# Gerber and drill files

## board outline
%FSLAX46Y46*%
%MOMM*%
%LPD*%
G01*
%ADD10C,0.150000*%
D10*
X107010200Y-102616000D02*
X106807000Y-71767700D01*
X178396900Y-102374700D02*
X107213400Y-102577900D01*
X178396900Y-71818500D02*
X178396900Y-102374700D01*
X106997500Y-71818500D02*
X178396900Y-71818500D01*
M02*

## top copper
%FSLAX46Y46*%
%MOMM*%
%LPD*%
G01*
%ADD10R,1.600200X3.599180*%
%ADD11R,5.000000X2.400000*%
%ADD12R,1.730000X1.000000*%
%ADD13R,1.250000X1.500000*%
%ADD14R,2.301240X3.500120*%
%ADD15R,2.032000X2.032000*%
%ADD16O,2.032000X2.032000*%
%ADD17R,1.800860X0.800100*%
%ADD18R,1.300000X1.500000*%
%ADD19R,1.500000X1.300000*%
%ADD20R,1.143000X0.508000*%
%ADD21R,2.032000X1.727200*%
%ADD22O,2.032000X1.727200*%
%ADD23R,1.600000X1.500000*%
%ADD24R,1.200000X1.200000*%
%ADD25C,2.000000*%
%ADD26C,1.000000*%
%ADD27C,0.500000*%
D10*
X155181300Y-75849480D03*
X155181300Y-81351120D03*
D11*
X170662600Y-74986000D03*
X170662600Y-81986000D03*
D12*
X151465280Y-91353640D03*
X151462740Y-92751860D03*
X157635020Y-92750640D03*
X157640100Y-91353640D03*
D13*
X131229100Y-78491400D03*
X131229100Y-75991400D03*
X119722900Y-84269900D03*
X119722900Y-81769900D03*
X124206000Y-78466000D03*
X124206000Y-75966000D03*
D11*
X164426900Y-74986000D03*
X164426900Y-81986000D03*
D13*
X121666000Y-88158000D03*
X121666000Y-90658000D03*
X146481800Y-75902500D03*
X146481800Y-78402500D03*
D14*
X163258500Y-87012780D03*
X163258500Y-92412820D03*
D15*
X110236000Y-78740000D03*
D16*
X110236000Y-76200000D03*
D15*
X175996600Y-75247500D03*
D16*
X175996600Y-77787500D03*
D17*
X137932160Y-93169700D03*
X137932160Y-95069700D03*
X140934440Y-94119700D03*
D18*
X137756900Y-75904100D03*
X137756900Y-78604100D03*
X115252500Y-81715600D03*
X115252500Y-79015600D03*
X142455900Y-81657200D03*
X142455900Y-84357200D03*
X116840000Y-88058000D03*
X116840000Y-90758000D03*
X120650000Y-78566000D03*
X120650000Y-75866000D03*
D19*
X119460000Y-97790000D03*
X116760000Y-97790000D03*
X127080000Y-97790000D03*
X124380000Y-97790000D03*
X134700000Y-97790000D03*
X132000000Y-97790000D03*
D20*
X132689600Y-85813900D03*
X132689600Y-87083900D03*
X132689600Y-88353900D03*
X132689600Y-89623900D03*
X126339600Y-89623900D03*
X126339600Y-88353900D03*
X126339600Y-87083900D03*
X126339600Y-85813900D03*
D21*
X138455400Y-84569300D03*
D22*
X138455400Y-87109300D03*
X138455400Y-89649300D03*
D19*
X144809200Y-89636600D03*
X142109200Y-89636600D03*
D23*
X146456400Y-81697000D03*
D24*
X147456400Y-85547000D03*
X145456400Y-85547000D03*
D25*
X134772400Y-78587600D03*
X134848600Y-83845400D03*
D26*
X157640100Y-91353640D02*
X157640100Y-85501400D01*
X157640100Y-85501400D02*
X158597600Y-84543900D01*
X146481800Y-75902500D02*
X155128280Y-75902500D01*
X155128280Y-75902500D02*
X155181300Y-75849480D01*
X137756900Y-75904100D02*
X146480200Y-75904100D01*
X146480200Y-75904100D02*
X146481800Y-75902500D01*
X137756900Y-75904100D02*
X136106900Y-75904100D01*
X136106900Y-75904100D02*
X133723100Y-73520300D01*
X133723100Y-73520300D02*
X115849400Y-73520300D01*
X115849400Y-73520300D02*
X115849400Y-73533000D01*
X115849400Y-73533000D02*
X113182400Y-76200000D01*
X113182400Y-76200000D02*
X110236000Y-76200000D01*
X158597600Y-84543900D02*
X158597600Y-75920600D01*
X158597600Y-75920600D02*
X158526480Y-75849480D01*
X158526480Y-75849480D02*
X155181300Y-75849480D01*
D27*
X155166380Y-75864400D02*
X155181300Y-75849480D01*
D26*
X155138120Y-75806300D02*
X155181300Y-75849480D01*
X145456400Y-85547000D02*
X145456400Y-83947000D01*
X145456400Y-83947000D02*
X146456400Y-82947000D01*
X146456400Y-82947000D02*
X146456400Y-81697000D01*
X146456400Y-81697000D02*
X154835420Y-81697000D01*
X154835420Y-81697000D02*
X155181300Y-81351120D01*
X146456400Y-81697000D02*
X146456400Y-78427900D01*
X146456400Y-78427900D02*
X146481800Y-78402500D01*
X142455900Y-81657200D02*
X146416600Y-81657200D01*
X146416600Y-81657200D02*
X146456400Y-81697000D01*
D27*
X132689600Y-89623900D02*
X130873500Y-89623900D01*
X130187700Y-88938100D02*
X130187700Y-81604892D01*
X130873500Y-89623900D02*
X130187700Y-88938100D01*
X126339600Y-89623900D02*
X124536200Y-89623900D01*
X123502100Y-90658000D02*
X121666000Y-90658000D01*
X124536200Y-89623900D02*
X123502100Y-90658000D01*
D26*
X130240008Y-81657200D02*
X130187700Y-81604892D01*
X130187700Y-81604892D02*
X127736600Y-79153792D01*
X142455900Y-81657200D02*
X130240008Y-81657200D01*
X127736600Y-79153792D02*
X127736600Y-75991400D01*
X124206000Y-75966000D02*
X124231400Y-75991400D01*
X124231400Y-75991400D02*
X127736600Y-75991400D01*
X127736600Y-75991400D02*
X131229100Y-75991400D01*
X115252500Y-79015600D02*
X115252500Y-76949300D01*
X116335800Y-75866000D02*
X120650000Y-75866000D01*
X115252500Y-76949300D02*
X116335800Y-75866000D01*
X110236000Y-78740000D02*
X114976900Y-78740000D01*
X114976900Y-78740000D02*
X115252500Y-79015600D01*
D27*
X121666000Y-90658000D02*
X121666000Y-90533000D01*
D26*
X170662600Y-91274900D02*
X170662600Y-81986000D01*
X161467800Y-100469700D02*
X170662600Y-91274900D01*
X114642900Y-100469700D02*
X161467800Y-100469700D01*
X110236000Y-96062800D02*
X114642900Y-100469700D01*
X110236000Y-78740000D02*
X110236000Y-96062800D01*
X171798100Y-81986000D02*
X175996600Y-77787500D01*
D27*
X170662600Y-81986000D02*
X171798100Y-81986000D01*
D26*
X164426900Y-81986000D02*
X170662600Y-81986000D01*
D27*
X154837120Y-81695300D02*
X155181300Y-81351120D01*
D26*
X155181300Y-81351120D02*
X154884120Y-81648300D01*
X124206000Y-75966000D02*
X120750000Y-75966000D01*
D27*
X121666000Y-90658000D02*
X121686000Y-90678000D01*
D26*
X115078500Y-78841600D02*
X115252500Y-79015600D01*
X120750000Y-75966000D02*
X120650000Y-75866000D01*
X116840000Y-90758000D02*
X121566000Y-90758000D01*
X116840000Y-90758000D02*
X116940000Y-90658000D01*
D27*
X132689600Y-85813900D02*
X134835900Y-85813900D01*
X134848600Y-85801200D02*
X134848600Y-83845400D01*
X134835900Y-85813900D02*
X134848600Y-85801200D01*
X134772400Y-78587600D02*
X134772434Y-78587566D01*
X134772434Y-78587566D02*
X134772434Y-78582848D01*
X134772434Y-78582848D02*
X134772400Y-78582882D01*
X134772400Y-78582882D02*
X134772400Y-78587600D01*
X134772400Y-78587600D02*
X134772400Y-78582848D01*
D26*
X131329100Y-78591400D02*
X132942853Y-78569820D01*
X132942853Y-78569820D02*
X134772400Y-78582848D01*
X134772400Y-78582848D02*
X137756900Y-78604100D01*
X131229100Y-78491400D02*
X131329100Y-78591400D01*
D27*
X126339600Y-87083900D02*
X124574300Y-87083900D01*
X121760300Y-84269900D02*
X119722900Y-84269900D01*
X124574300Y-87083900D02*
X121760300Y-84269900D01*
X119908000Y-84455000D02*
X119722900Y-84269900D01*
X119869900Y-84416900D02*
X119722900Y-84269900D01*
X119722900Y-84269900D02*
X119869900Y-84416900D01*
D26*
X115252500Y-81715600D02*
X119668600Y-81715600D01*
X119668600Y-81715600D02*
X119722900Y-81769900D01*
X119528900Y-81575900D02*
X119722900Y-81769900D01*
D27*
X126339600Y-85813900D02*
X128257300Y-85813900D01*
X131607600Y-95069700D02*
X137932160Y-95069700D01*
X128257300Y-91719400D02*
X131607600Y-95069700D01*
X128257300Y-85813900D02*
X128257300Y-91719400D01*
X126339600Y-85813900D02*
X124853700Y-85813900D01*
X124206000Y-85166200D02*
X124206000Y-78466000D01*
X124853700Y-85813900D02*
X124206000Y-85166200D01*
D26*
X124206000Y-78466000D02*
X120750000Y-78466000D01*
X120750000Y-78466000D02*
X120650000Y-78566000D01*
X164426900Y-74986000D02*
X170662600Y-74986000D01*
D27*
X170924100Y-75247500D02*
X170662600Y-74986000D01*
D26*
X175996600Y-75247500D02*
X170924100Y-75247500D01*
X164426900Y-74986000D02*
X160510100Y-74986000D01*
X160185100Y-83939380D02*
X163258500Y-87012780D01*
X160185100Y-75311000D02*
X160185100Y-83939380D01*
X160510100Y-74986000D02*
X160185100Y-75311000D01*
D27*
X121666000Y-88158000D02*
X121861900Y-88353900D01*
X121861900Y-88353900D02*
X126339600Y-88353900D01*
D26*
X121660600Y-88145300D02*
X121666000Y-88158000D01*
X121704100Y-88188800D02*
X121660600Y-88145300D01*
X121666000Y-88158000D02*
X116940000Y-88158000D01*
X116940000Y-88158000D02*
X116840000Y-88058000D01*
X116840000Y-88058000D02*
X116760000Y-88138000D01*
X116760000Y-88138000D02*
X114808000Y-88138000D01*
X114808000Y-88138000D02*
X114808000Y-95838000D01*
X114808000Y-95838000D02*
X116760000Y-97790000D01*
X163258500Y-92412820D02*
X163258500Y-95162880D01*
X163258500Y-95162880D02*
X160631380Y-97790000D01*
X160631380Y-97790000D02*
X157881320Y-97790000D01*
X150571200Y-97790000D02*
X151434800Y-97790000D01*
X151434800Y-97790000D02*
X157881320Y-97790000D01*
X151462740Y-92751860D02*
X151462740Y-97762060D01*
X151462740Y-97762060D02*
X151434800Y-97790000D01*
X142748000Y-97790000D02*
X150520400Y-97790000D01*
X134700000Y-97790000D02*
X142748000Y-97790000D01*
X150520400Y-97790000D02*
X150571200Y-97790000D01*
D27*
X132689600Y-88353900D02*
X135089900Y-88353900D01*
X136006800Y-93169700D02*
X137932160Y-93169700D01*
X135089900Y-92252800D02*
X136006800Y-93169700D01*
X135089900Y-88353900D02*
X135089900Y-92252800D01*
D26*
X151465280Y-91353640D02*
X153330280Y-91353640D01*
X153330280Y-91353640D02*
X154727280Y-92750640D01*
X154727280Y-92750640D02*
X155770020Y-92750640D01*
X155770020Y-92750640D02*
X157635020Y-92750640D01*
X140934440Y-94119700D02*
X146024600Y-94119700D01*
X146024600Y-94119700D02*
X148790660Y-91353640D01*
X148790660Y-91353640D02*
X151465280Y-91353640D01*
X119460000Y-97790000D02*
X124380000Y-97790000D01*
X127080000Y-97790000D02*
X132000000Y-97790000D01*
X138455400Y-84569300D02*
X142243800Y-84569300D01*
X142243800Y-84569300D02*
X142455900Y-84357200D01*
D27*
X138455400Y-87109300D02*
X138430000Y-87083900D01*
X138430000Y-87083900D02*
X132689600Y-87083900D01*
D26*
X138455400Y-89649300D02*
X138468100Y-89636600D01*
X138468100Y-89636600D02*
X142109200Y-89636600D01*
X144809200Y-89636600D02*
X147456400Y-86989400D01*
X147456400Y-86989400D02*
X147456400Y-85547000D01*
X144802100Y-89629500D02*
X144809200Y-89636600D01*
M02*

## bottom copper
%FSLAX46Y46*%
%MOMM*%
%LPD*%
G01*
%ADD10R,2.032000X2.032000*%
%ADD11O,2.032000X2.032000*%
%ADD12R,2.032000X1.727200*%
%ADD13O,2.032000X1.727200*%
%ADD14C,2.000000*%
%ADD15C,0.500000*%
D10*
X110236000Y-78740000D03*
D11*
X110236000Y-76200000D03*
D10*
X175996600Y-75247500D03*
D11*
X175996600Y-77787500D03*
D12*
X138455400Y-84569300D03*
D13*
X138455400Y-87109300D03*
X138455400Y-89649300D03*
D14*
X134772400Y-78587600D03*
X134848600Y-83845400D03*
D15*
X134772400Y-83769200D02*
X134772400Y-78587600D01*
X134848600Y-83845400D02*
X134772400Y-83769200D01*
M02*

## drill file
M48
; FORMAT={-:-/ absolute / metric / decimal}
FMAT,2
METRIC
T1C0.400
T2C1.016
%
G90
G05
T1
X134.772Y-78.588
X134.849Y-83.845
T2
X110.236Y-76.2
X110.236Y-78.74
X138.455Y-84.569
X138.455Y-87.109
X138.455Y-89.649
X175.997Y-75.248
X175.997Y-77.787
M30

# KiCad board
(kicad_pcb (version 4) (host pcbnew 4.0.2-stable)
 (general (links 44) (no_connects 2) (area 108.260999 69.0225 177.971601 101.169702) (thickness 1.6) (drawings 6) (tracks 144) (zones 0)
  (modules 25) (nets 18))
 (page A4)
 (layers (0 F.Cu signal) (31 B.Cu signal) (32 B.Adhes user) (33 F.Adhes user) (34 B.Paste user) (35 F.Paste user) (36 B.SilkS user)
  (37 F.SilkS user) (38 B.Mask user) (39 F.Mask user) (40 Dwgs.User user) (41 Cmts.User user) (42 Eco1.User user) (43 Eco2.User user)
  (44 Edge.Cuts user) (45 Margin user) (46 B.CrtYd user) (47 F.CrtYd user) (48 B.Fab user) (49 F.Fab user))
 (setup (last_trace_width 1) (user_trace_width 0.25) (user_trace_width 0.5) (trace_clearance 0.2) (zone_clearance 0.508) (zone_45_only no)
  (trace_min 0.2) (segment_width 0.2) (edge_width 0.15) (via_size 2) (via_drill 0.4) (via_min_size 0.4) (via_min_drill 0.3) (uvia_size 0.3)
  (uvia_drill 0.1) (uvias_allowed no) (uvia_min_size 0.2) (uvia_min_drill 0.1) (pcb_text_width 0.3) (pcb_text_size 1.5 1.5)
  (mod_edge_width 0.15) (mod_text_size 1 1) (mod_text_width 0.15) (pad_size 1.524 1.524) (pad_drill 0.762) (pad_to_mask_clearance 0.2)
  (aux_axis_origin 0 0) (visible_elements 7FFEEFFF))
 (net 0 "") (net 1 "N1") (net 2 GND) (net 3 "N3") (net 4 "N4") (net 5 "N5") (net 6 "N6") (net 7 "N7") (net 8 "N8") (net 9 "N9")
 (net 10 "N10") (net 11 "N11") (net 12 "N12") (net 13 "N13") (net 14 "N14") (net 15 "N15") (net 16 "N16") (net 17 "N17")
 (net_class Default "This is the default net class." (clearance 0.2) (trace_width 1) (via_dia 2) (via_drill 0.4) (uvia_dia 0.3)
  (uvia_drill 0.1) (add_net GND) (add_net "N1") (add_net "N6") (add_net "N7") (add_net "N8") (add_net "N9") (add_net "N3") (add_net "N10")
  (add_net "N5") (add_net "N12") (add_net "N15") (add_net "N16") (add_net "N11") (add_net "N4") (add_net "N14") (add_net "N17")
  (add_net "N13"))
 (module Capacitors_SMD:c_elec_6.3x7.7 (layer F.Cu) (at 155.1813 78.6003 90)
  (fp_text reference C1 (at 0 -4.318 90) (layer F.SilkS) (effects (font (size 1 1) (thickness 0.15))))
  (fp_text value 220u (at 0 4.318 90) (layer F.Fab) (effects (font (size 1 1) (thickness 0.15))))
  (pad 1 smd rect (at 2.75082 0 90) (size 3.59918 1.6002) (layers F.Cu F.Paste F.Mask) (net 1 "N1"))
  (pad 2 smd rect (at -2.75082 0 90) (size 3.59918 1.6002) (layers F.Cu F.Paste F.Mask) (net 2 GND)))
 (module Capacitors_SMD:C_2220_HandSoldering (layer F.Cu) (at 170.6626 78.486 270)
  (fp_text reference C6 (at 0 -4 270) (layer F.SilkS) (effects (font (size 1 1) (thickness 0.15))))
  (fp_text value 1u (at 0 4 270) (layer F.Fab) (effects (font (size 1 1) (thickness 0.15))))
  (pad 1 smd rect (at -3.5 0 270) (size 2.4 5) (layers F.Cu F.Paste F.Mask) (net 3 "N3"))
  (pad 2 smd rect (at 3.5 0 270) (size 2.4 5) (layers F.Cu F.Paste F.Mask) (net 2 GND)))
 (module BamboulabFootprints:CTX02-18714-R (layer F.Cu) (at 154.6352 91.9988)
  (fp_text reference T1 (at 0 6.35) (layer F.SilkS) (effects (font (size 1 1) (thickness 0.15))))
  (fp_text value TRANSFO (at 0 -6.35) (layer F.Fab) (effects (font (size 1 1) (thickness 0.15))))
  (pad 1 smd rect (at -3.16992 -0.64516) (size 1.73 1) (layers F.Cu F.Paste F.Mask) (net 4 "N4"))
  (pad 2 smd rect (at -3.17246 0.75306) (size 1.73 1) (layers F.Cu F.Paste F.Mask) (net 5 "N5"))
  (pad 4 smd rect (at 2.99982 0.75184) (size 1.73 1) (layers F.Cu F.Paste F.Mask) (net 4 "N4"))
  (pad 3 smd rect (at 3.0049 -0.64516) (size 1.73 1) (layers F.Cu F.Paste F.Mask) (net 1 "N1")))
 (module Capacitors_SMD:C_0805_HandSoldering (layer F.Cu) (at 131.2291 77.2414 90)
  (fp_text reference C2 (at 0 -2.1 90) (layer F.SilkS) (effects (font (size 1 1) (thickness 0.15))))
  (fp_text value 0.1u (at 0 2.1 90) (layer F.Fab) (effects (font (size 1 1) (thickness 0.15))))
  (pad 1 smd rect (at -1.25 0 90) (size 1.5 1.25) (layers F.Cu F.Paste F.Mask) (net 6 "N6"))
  (pad 2 smd rect (at 1.25 0 90) (size 1.5 1.25) (layers F.Cu F.Paste F.Mask) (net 2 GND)))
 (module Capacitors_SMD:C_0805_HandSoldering (layer F.Cu) (at 119.7229 83.0199 90)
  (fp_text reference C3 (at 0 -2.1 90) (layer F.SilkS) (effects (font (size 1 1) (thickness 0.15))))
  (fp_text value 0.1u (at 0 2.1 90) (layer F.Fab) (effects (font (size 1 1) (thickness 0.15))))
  (pad 1 smd rect (at -1.25 0 90) (size 1.5 1.25) (layers F.Cu F.Paste F.Mask) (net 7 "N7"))
  (pad 2 smd rect (at 1.25 0 90) (size 1.5 1.25) (layers F.Cu F.Paste F.Mask) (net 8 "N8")))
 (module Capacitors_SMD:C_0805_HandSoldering (layer F.Cu) (at 124.206 77.216 90)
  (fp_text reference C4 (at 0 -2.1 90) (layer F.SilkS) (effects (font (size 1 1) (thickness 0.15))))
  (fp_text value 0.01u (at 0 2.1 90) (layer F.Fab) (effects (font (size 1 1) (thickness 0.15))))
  (pad 1 smd rect (at -1.25 0 90) (size 1.5 1.25) (layers F.Cu F.Paste F.Mask) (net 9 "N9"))
  (pad 2 smd rect (at 1.25 0 90) (size 1.5 1.25) (layers F.Cu F.Paste F.Mask) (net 2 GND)))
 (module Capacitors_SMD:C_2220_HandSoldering (layer F.Cu) (at 164.4269 78.486 270)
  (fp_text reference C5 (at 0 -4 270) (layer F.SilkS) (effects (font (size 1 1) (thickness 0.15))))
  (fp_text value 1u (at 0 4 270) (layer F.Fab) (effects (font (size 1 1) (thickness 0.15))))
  (pad 1 smd rect (at -3.5 0 270) (size 2.4 5) (layers F.Cu F.Paste F.Mask) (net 3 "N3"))
  (pad 2 smd rect (at 3.5 0 270) (size 2.4 5) (layers F.Cu F.Paste F.Mask) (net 2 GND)))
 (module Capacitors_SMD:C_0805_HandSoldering (layer F.Cu) (at 121.666 89.408 270)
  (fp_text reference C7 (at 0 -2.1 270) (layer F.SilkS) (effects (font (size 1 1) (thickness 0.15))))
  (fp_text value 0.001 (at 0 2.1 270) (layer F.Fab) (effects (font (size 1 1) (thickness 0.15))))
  (pad 1 smd rect (at -1.25 0 270) (size 1.5 1.25) (layers F.Cu F.Paste F.Mask) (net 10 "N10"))
  (pad 2 smd rect (at 1.25 0 270) (size 1.5 1.25) (layers F.Cu F.Paste F.Mask) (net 2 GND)))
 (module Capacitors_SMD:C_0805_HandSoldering (layer F.Cu) (at 146.4818 77.1525 270)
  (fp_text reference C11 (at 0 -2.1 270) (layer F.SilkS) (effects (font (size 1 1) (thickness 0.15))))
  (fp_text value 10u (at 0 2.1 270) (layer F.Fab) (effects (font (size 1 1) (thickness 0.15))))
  (pad 1 smd rect (at -1.25 0 270) (size 1.5 1.25) (layers F.Cu F.Paste F.Mask) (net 1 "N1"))
  (pad 2 smd rect (at 1.25 0 270) (size 1.5 1.25) (layers F.Cu F.Paste F.Mask) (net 2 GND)))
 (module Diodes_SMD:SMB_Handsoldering (layer F.Cu) (at 163.2585 89.7128 270)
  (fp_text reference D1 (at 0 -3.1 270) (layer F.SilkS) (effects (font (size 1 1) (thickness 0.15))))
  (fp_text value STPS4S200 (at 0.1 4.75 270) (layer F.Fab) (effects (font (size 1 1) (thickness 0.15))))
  (pad 1 smd rect (at -2.70002 0 270) (size 3.50012 2.30124) (layers F.Cu F.Paste F.Mask) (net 3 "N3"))
  (pad 2 smd rect (at 2.70002 0 270) (size 3.50012 2.30124) (layers F.Cu F.Paste F.Mask) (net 5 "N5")))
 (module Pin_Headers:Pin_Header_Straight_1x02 (layer F.Cu) (at 110.236 78.74 180)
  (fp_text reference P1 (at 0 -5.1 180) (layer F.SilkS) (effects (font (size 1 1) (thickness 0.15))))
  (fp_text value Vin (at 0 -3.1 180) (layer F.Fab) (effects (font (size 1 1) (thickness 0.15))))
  (pad 1 thru_hole rect (at 0 0 180) (size 2.032 2.032) (drill 1.016) (layers *.Cu *.Mask F.SilkS) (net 2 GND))
  (pad 2 thru_hole oval (at 0 2.54 180) (size 2.032 2.032) (drill 1.016) (layers *.Cu *.Mask F.SilkS) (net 1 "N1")))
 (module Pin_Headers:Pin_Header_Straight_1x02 (layer F.Cu) (at 175.9966 75.2475)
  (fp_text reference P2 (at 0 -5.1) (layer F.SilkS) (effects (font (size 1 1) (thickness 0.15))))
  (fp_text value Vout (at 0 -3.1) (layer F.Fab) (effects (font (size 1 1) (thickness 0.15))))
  (pad 1 thru_hole rect (at 0 0) (size 2.032 2.032) (drill 1.016) (layers *.Cu *.Mask F.SilkS) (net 3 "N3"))
  (pad 2 thru_hole oval (at 0 2.54) (size 2.032 2.032) (drill 1.016) (layers *.Cu *.Mask F.SilkS) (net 2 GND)))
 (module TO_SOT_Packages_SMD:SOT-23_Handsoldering (layer F.Cu) (at 139.4333 94.1197 270)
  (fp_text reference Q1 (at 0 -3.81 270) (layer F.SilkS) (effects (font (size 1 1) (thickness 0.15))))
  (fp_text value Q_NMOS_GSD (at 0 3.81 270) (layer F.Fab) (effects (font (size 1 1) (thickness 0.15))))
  (pad 1 smd rect (at -0.95 1.50114 270) (size 0.8001 1.80086) (layers F.Cu F.Paste F.Mask) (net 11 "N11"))
  (pad 2 smd rect (at 0.95 1.50114 270) (size 0.8001 1.80086) (layers F.Cu F.Paste F.Mask) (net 9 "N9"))
  (pad 3 smd rect (at 0 -1.50114 270) (size 0.8001 1.80086) (layers F.Cu F.Paste F.Mask) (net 4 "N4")))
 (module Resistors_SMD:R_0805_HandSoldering (layer F.Cu) (at 137.7569 77.2541 270)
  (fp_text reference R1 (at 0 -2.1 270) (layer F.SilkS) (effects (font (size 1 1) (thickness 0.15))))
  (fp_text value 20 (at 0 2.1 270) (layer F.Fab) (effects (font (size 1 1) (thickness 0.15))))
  (pad 1 smd rect (at -1.35 0 270) (size 1.5 1.3) (layers F.Cu F.Paste F.Mask) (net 1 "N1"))
  (pad 2 smd rect (at 1.35 0 270) (size 1.5 1.3) (layers F.Cu F.Paste F.Mask) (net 6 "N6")))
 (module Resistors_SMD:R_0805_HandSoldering (layer F.Cu) (at 115.2525 80.3656 90)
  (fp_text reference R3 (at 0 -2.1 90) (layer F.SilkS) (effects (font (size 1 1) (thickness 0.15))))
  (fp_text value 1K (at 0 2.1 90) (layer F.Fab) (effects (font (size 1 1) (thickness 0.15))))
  (pad 1 smd rect (at -1.35 0 90) (size 1.5 1.3) (layers F.Cu F.Paste F.Mask) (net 8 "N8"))
  (pad 2 smd rect (at 1.35 0 90) (size 1.5 1.3) (layers F.Cu F.Paste F.Mask) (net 2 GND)))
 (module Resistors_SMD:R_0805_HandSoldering (layer F.Cu) (at 142.4559 83.0072 270)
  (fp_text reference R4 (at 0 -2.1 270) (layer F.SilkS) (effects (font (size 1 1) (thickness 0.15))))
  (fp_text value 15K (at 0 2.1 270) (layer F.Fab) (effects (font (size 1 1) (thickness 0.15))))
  (pad 1 smd rect (at -1.35 0 270) (size 1.5 1.3) (layers F.Cu F.Paste F.Mask) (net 2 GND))
  (pad 2 smd rect (at 1.35 0 270) (size 1.5 1.3) (layers F.Cu F.Paste F.Mask) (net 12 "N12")))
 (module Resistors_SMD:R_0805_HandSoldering (layer F.Cu) (at 116.84 89.408 270)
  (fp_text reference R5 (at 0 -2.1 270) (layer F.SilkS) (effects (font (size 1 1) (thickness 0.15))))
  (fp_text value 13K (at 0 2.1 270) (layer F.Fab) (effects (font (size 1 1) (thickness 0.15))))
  (pad 1 smd rect (at -1.35 0 270) (size 1.5 1.3) (layers F.Cu F.Paste F.Mask) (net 10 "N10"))
  (pad 2 smd rect (at 1.35 0 270) (size 1.5 1.3) (layers F.Cu F.Paste F.Mask) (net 2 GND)))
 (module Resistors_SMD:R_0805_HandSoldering (layer F.Cu) (at 120.65 77.216 90)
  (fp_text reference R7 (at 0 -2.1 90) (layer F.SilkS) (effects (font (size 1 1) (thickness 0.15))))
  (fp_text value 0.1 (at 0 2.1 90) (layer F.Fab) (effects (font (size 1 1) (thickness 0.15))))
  (pad 1 smd rect (at -1.35 0 90) (size 1.5 1.3) (layers F.Cu F.Paste F.Mask) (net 9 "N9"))
  (pad 2 smd rect (at 1.35 0 90) (size 1.5 1.3) (layers F.Cu F.Paste F.Mask) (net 2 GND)))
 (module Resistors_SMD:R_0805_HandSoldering (layer F.Cu) (at 118.11 97.79 180)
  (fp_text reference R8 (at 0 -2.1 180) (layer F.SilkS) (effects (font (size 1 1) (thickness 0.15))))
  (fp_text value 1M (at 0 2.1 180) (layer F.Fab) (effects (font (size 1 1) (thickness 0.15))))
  (pad 1 smd rect (at -1.35 0 180) (size 1.5 1.3) (layers F.Cu F.Paste F.Mask) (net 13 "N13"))
  (pad 2 smd rect (at 1.35 0 180) (size 1.5 1.3) (layers F.Cu F.Paste F.Mask) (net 10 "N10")))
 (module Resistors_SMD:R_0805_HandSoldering (layer F.Cu) (at 125.73 97.79 180)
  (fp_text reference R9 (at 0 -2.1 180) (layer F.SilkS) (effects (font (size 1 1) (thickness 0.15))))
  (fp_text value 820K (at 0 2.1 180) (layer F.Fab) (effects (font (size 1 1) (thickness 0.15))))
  (pad 1 smd rect (at -1.35 0 180) (size 1.5 1.3) (layers F.Cu F.Paste F.Mask) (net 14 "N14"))
  (pad 2 smd rect (at 1.35 0 180) (size 1.5 1.3) (layers F.Cu F.Paste F.Mask) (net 13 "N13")))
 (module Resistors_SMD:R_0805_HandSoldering (layer F.Cu) (at 133.35 97.79 180)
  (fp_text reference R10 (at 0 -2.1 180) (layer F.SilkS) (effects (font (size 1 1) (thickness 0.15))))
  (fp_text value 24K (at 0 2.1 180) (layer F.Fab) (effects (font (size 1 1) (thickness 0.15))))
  (pad 1 smd rect (at -1.35 0 180) (size 1.5 1.3) (layers F.Cu F.Paste F.Mask) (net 5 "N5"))
  (pad 2 smd rect (at 1.35 0 180) (size 1.5 1.3) (layers F.Cu F.Paste F.Mask) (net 14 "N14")))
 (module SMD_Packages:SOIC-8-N (layer F.Cu) (at 129.5146 87.7189 270)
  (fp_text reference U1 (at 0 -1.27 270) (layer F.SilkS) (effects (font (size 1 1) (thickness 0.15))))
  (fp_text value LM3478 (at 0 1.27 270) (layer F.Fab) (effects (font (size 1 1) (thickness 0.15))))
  (pad 8 smd rect (at -1.905 -3.175 270) (size 0.508 1.143) (layers F.Cu F.Paste F.Mask) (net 6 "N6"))
  (pad 7 smd rect (at -0.635 -3.175 270) (size 0.508 1.143) (layers F.Cu F.Paste F.Mask) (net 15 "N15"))
  (pad 6 smd rect (at 0.635 -3.175 270) (size 0.508 1.143) (layers F.Cu F.Paste F.Mask) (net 11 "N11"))
  (pad 5 smd rect (at 1.905 -3.175 270) (size 0.508 1.143) (layers F.Cu F.Paste F.Mask) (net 2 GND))
  (pad 4 smd rect (at 1.905 3.175 270) (size 0.508 1.143) (layers F.Cu F.Paste F.Mask) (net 2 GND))
  (pad 3 smd rect (at 0.635 3.175 270) (size 0.508 1.143) (layers F.Cu F.Paste F.Mask) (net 10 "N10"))
  (pad 2 smd rect (at -0.635 3.175 270) (size 0.508 1.143) (layers F.Cu F.Paste F.Mask) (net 7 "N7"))
  (pad 1 smd rect (at -1.905 3.175 270) (size 0.508 1.143) (layers F.Cu F.Paste F.Mask) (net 9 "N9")))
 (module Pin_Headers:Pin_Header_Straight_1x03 (layer F.Cu) (at 138.4554 84.5693)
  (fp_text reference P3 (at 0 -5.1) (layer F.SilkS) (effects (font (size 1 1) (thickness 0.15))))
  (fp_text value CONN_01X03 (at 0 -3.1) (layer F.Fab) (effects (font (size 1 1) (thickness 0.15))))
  (pad 1 thru_hole rect (at 0 0) (size 2.032 1.7272) (drill 1.016) (layers *.Cu *.Mask F.SilkS) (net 12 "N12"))
  (pad 2 thru_hole oval (at 0 2.54) (size 2.032 1.7272) (drill 1.016) (layers *.Cu *.Mask F.SilkS) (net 15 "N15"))
  (pad 3 thru_hole oval (at 0 5.08) (size 2.032 1.7272) (drill 1.016) (layers *.Cu *.Mask F.SilkS) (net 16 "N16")))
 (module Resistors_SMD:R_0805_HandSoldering (layer F.Cu) (at 143.4592 89.6366 180)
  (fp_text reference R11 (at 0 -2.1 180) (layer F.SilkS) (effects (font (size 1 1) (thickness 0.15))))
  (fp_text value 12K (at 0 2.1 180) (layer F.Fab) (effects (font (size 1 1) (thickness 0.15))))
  (pad 1 smd rect (at -1.35 0 180) (size 1.5 1.3) (layers F.Cu F.Paste F.Mask) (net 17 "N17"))
  (pad 2 smd rect (at 1.35 0 180) (size 1.5 1.3) (layers F.Cu F.Paste F.Mask) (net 16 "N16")))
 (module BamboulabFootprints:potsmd (layer F.Cu) (at 146.4564 83.947)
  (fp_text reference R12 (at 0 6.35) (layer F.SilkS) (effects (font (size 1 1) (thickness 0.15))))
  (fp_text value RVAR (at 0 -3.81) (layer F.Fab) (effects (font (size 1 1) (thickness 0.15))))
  (pad 1 smd rect (at 0 -2.25) (size 1.6 1.5) (layers F.Cu F.Paste F.Mask) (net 2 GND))
  (pad 2 smd rect (at 1 1.6) (size 1.2 1.2) (layers F.Cu F.Paste F.Mask) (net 17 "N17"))
  (pad 1 smd rect (at -1 1.6) (size 1.2 1.2) (layers F.Cu F.Paste F.Mask) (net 2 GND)))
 (gr_line (start 107.0102 102.616) (end 106.807 71.7677) (layer Edge.Cuts) (width 0.15))
 (gr_line (start 178.3969 102.3747) (end 107.2134 102.5779) (layer Edge.Cuts) (width 0.15))
 (gr_line (start 178.3969 71.8185) (end 178.3969 102.3747) (layer Edge.Cuts) (width 0.15))
 (gr_line (start 106.9975 71.8185) (end 178.3969 71.8185) (layer Edge.Cuts) (width 0.15))
 (segment (start 157.6401 91.35364) (end 157.6401 85.5014) (width 1) (layer F.Cu) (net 1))
 (segment (start 157.6401 85.5014) (end 158.5976 84.5439) (width 1) (layer F.Cu) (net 1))
 (segment (start 146.4818 75.9025) (end 155.12828 75.9025) (width 1) (layer F.Cu) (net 1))
 (segment (start 155.12828 75.9025) (end 155.1813 75.84948) (width 1) (layer F.Cu) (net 1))
 (segment (start 137.7569 75.9041) (end 146.4802 75.9041) (width 1) (layer F.Cu) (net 1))
 (segment (start 146.4802 75.9041) (end 146.4818 75.9025) (width 1) (layer F.Cu) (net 1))
 (segment (start 137.7569 75.9041) (end 136.1069 75.9041) (width 1) (layer F.Cu) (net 1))
 (segment (start 136.1069 75.9041) (end 133.7231 73.5203) (width 1) (layer F.Cu) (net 1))
 (segment (start 133.7231 73.5203) (end 115.8494 73.5203) (width 1) (layer F.Cu) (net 1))
 (segment (start 115.8494 73.5203) (end 115.8494 73.533) (width 1) (layer F.Cu) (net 1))
 (segment (start 115.8494 73.533) (end 113.1824 76.2) (width 1) (layer F.Cu) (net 1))
 (segment (start 113.1824 76.2) (end 110.236 76.2) (width 1) (layer F.Cu) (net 1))
 (segment (start 158.5976 84.5439) (end 158.5976 75.9206) (width 1) (layer F.Cu) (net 1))
 (segment (start 158.5976 75.9206) (end 158.52648 75.84948) (width 1) (layer F.Cu) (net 1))
 (segment (start 158.52648 75.84948) (end 155.1813 75.84948) (width 1) (layer F.Cu) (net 1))
 (segment (start 155.16638 75.8644) (end 155.1813 75.84948) (width 0.5) (layer F.Cu) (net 1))
 (segment (start 155.13812 75.8063) (end 155.1813 75.84948) (width 1) (layer F.Cu) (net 1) (status 30))
 (segment (start 145.4564 85.547) (end 145.4564 83.947) (width 1) (layer F.Cu) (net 2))
 (segment (start 145.4564 83.947) (end 146.4564 82.947) (width 1) (layer F.Cu) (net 2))
 (segment (start 146.4564 82.947) (end 146.4564 81.697) (width 1) (layer F.Cu) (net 2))
 (segment (start 146.4564 81.697) (end 154.83542 81.697) (width 1) (layer F.Cu) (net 2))
 (segment (start 154.83542 81.697) (end 155.1813 81.35112) (width 1) (layer F.Cu) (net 2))
 (segment (start 146.4564 81.697) (end 146.4564 78.4279) (width 1) (layer F.Cu) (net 2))
 (segment (start 146.4564 78.4279) (end 146.4818 78.4025) (width 1) (layer F.Cu) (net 2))
 (segment (start 142.4559 81.6572) (end 146.4166 81.6572) (width 1) (layer F.Cu) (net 2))
 (segment (start 146.4166 81.6572) (end 146.4564 81.697) (width 1) (layer F.Cu) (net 2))
 (segment (start 132.6896 89.6239) (end 130.8735 89.6239) (width 0.5) (layer F.Cu) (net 2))
 (segment (start 130.1877 88.9381) (end 130.1877 81.604892) (width 0.5) (layer F.Cu) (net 2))
 (segment (start 130.8735 89.6239) (end 130.1877 88.9381) (width 0.5) (layer F.Cu) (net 2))
 (segment (start 126.3396 89.6239) (end 124.5362 89.6239) (width 0.5) (layer F.Cu) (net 2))
 (segment (start 123.5021 90.658) (end 121.666 90.658) (width 0.5) (layer F.Cu) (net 2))
 (segment (start 124.5362 89.6239) (end 123.5021 90.658) (width 0.5) (layer F.Cu) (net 2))
 (segment (start 130.240008 81.6572) (end 130.1877 81.604892) (width 1) (layer F.Cu) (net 2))
 (segment (start 130.1877 81.604892) (end 127.7366 79.153792) (width 1) (layer F.Cu) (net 2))
 (segment (start 142.4559 81.6572) (end 130.240008 81.6572) (width 1) (layer F.Cu) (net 2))
 (segment (start 127.7366 79.153792) (end 127.7366 75.9914) (width 1) (layer F.Cu) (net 2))
 (segment (start 124.206 75.966) (end 124.2314 75.9914) (width 1) (layer F.Cu) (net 2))
 (segment (start 124.2314 75.9914) (end 127.7366 75.9914) (width 1) (layer F.Cu) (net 2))
 (segment (start 127.7366 75.9914) (end 131.2291 75.9914) (width 1) (layer F.Cu) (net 2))
 (segment (start 115.2525 79.0156) (end 115.2525 76.9493) (width 1) (layer F.Cu) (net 2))
 (segment (start 116.3358 75.866) (end 120.65 75.866) (width 1) (layer F.Cu) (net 2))
 (segment (start 115.2525 76.9493) (end 116.3358 75.866) (width 1) (layer F.Cu) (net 2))
 (segment (start 110.236 78.74) (end 114.9769 78.74) (width 1) (layer F.Cu) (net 2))
 (segment (start 114.9769 78.74) (end 115.2525 79.0156) (width 1) (layer F.Cu) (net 2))
 (segment (start 121.666 90.658) (end 121.666 90.533) (width 0.5) (layer F.Cu) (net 2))
 (segment (start 170.6626 91.2749) (end 170.6626 81.986) (width 1) (layer F.Cu) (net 2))
 (segment (start 161.4678 100.4697) (end 170.6626 91.2749) (width 1) (layer F.Cu) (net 2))
 (segment (start 114.6429 100.4697) (end 161.4678 100.4697) (width 1) (layer F.Cu) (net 2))
 (segment (start 110.236 96.0628) (end 114.6429 100.4697) (width 1) (layer F.Cu) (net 2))
 (segment (start 110.236 78.74) (end 110.236 96.0628) (width 1) (layer F.Cu) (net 2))
 (segment (start 171.7981 81.986) (end 175.9966 77.7875) (width 1) (layer F.Cu) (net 2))
 (segment (start 170.6626 81.986) (end 171.7981 81.986) (width 0.5) (layer F.Cu) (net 2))
 (segment (start 164.4269 81.986) (end 170.6626 81.986) (width 1) (layer F.Cu) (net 2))
 (segment (start 154.83712 81.6953) (end 155.1813 81.35112) (width 0.5) (layer F.Cu) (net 2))
 (segment (start 155.1813 81.35112) (end 154.88412 81.6483) (width 1) (layer F.Cu) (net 2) (status 30))
 (segment (start 124.206 75.966) (end 120.75 75.966) (width 1) (layer F.Cu) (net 2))
 (segment (start 121.666 90.658) (end 121.686 90.678) (width 0.5) (layer F.Cu) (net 2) (status 30))
 (segment (start 115.0785 78.8416) (end 115.2525 79.0156) (width 1) (layer F.Cu) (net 2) (status 30))
 (segment (start 120.75 75.966) (end 120.65 75.866) (width 1) (layer F.Cu) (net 2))
 (segment (start 116.84 90.758) (end 121.566 90.758) (width 1) (layer F.Cu) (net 2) (status 20))
 (segment (start 116.84 90.758) (end 116.94 90.658) (width 1) (layer F.Cu) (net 2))
 (segment (start 132.6896 85.8139) (end 134.8359 85.8139) (width 0.5) (layer F.Cu) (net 6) (status 400000))
 (via (at 134.7724 78.5876) (size 2) (drill 0.4) (layers F.Cu B.Cu) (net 6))
 (segment (start 134.7724 83.7692) (end 134.7724 78.5876) (width 0.5) (layer B.Cu) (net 6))
 (segment (start 134.8486 83.8454) (end 134.7724 83.7692) (width 0.5) (layer B.Cu) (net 6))
 (via (at 134.8486 83.8454) (size 2) (drill 0.4) (layers F.Cu B.Cu) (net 6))
 (segment (start 134.8486 85.8012) (end 134.8486 83.8454) (width 0.5) (layer F.Cu) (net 6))
 (segment (start 134.8359 85.8139) (end 134.8486 85.8012) (width 0.5) (layer F.Cu) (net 6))
 (segment (start 134.7724 78.5876) (end 134.772434 78.587566) (width 0.5) (layer F.Cu) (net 6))
 (segment (start 134.772434 78.587566) (end 134.772434 78.582848) (width 0.5) (layer F.Cu) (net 6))
 (segment (start 134.772434 78.582848) (end 134.7724 78.582882) (width 0.5) (layer F.Cu) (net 6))
 (segment (start 134.7724 78.582882) (end 134.7724 78.5876) (width 0.5) (layer F.Cu) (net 6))
 (segment (start 134.7724 78.5876) (end 134.7724 78.582848) (width 0.5) (layer F.Cu) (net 6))
 (segment (start 131.3291 78.5914) (end 132.942853 78.56982) (width 1) (layer F.Cu) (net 6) (status 10))
 (segment (start 132.942853 78.56982) (end 134.7724 78.582848) (width 1) (layer F.Cu) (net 6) (status 20))
 (segment (start 134.7724 78.582848) (end 137.7569 78.6041) (width 1) (layer F.Cu) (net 6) (status 20))
 (segment (start 131.2291 78.4914) (end 131.3291 78.5914) (width 1) (layer F.Cu) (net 6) (status 30))
 (segment (start 126.3396 87.0839) (end 124.5743 87.0839) (width 0.5) (layer F.Cu) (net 7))
 (segment (start 121.7603 84.2699) (end 119.7229 84.2699) (width 0.5) (layer F.Cu) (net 7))
 (segment (start 124.5743 87.0839) (end 121.7603 84.2699) (width 0.5) (layer F.Cu) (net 7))
 (segment (start 119.908 84.455) (end 119.7229 84.2699) (width 0.5) (layer F.Cu) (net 7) (status 30))
 (segment (start 119.8699 84.4169) (end 119.7229 84.2699) (width 0.5) (layer F.Cu) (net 7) (status 30))
 (segment (start 119.7229 84.2699) (end 119.8699 84.4169) (width 0.5) (layer F.Cu) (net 7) (status 30))
 (segment (start 115.2525 81.7156) (end 119.6686 81.7156) (width 1) (layer F.Cu) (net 8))
 (segment (start 119.6686 81.7156) (end 119.7229 81.7699) (width 1) (layer F.Cu) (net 8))
 (segment (start 119.5289 81.5759) (end 119.7229 81.7699) (width 1) (layer F.Cu) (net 8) (status 30))
 (segment (start 126.3396 85.8139) (end 128.2573 85.8139) (width 0.5) (layer F.Cu) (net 9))
 (segment (start 131.6076 95.0697) (end 137.93216 95.0697) (width 0.5) (layer F.Cu) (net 9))
 (segment (start 128.2573 91.7194) (end 131.6076 95.0697) (width 0.5) (layer F.Cu) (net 9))
 (segment (start 128.2573 85.8139) (end 128.2573 91.7194) (width 0.5) (layer F.Cu) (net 9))
 (segment (start 126.3396 85.8139) (end 124.8537 85.8139) (width 0.5) (layer F.Cu) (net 9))
 (segment (start 124.206 85.1662) (end 124.206 78.466) (width 0.5) (layer F.Cu) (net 9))
 (segment (start 124.8537 85.8139) (end 124.206 85.1662) (width 0.5) (layer F.Cu) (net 9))
 (segment (start 124.206 78.466) (end 120.75 78.466) (width 1) (layer F.Cu) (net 9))
 (segment (start 120.75 78.466) (end 120.65 78.566) (width 1) (layer F.Cu) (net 9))
 (segment (start 164.4269 74.986) (end 170.6626 74.986) (width 1) (layer F.Cu) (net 3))
 (segment (start 170.9241 75.2475) (end 170.6626 74.986) (width 0.5) (layer F.Cu) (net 3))
 (segment (start 175.9966 75.2475) (end 170.9241 75.2475) (width 1) (layer F.Cu) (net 3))
 (segment (start 164.4269 74.986) (end 160.5101 74.986) (width 1) (layer F.Cu) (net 3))
 (segment (start 160.1851 83.93938) (end 163.2585 87.01278) (width 1) (layer F.Cu) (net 3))
 (segment (start 160.1851 75.311) (end 160.1851 83.93938) (width 1) (layer F.Cu) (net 3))
 (segment (start 160.5101 74.986) (end 160.1851 75.311) (width 1) (layer F.Cu) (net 3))
 (segment (start 121.666 88.158) (end 121.8619 88.3539) (width 0.5) (layer F.Cu) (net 10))
 (segment (start 121.8619 88.3539) (end 126.3396 88.3539) (width 0.5) (layer F.Cu) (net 10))
 (segment (start 121.6606 88.1453) (end 121.666 88.158) (width 1) (layer F.Cu) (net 10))
 (segment (start 121.7041 88.1888) (end 121.6606 88.1453) (width 1) (layer F.Cu) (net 10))
 (segment (start 121.666 88.158) (end 116.94 88.158) (width 1) (layer F.Cu) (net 10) (status 10))
 (segment (start 116.94 88.158) (end 116.84 88.058) (width 1) (layer F.Cu) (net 10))
 (segment (start 116.84 88.058) (end 116.76 88.138) (width 1) (layer F.Cu) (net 10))
 (segment (start 116.76 88.138) (end 114.808 88.138) (width 1) (layer F.Cu) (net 10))
 (segment (start 114.808 88.138) (end 114.808 95.838) (width 1) (layer F.Cu) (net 10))
 (segment (start 114.808 95.838) (end 116.76 97.79) (width 1) (layer F.Cu) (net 10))
 (segment (start 163.2585 92.41282) (end 163.2585 95.16288) (width 1) (layer F.Cu) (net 5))
 (segment (start 163.2585 95.16288) (end 160.63138 97.79) (width 1) (layer F.Cu) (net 5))
 (segment (start 160.63138 97.79) (end 157.88132 97.79) (width 1) (layer F.Cu) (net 5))
 (segment (start 150.5712 97.79) (end 151.4348 97.79) (width 1) (layer F.Cu) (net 5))
 (segment (start 151.4348 97.79) (end 157.88132 97.79) (width 1) (layer F.Cu) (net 5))
 (segment (start 151.46274 92.75186) (end 151.46274 97.76206) (width 1) (layer F.Cu) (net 5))
 (segment (start 151.46274 97.76206) (end 151.4348 97.79) (width 1) (layer F.Cu) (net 5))
 (segment (start 142.748 97.79) (end 150.5204 97.79) (width 1) (layer F.Cu) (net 5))
 (segment (start 134.7 97.79) (end 142.748 97.79) (width 1) (layer F.Cu) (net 5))
 (segment (start 150.5204 97.79) (end 150.5712 97.79) (width 1) (layer F.Cu) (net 5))
 (segment (start 132.6896 88.3539) (end 135.0899 88.3539) (width 0.5) (layer F.Cu) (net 11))
 (segment (start 136.0068 93.1697) (end 137.93216 93.1697) (width 0.5) (layer F.Cu) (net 11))
 (segment (start 135.0899 92.2528) (end 136.0068 93.1697) (width 0.5) (layer F.Cu) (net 11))
 (segment (start 135.0899 88.3539) (end 135.0899 92.2528) (width 0.5) (layer F.Cu) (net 11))
 (segment (start 151.46528 91.35364) (end 153.33028 91.35364) (width 1) (layer F.Cu) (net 4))
 (segment (start 153.33028 91.35364) (end 154.72728 92.75064) (width 1) (layer F.Cu) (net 4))
 (segment (start 154.72728 92.75064) (end 155.77002 92.75064) (width 1) (layer F.Cu) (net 4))
 (segment (start 155.77002 92.75064) (end 157.63502 92.75064) (width 1) (layer F.Cu) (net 4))
 (segment (start 140.93444 94.1197) (end 146.0246 94.1197) (width 1) (layer F.Cu) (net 4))
 (segment (start 146.0246 94.1197) (end 148.79066 91.35364) (width 1) (layer F.Cu) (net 4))
 (segment (start 148.79066 91.35364) (end 151.46528 91.35364) (width 1) (layer F.Cu) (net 4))
 (segment (start 119.46 97.79) (end 124.38 97.79) (width 1) (layer F.Cu) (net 13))
 (segment (start 127.08 97.79) (end 132 97.79) (width 1) (layer F.Cu) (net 14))
 (segment (start 138.4554 84.5693) (end 142.2438 84.5693) (width 1) (layer F.Cu) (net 12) (status 10))
 (segment (start 142.2438 84.5693) (end 142.4559 84.3572) (width 1) (layer F.Cu) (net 12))
 (segment (start 138.4554 87.1093) (end 138.43 87.0839) (width 0.5) (layer F.Cu) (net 15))
 (segment (start 138.43 87.0839) (end 132.6896 87.0839) (width 0.5) (layer F.Cu) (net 15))
 (segment (start 138.4554 89.6493) (end 138.4681 89.6366) (width 1) (layer F.Cu) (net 16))
 (segment (start 138.4681 89.6366) (end 142.1092 89.6366) (width 1) (layer F.Cu) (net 16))
 (segment (start 144.8092 89.6366) (end 147.4564 86.9894) (width 1) (layer F.Cu) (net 17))
 (segment (start 147.4564 86.9894) (end 147.4564 85.547) (width 1) (layer F.Cu) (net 17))
 (segment (start 144.8021 89.6295) (end 144.8092 89.6366) (width 1) (layer F.Cu) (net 17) (status 30)))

